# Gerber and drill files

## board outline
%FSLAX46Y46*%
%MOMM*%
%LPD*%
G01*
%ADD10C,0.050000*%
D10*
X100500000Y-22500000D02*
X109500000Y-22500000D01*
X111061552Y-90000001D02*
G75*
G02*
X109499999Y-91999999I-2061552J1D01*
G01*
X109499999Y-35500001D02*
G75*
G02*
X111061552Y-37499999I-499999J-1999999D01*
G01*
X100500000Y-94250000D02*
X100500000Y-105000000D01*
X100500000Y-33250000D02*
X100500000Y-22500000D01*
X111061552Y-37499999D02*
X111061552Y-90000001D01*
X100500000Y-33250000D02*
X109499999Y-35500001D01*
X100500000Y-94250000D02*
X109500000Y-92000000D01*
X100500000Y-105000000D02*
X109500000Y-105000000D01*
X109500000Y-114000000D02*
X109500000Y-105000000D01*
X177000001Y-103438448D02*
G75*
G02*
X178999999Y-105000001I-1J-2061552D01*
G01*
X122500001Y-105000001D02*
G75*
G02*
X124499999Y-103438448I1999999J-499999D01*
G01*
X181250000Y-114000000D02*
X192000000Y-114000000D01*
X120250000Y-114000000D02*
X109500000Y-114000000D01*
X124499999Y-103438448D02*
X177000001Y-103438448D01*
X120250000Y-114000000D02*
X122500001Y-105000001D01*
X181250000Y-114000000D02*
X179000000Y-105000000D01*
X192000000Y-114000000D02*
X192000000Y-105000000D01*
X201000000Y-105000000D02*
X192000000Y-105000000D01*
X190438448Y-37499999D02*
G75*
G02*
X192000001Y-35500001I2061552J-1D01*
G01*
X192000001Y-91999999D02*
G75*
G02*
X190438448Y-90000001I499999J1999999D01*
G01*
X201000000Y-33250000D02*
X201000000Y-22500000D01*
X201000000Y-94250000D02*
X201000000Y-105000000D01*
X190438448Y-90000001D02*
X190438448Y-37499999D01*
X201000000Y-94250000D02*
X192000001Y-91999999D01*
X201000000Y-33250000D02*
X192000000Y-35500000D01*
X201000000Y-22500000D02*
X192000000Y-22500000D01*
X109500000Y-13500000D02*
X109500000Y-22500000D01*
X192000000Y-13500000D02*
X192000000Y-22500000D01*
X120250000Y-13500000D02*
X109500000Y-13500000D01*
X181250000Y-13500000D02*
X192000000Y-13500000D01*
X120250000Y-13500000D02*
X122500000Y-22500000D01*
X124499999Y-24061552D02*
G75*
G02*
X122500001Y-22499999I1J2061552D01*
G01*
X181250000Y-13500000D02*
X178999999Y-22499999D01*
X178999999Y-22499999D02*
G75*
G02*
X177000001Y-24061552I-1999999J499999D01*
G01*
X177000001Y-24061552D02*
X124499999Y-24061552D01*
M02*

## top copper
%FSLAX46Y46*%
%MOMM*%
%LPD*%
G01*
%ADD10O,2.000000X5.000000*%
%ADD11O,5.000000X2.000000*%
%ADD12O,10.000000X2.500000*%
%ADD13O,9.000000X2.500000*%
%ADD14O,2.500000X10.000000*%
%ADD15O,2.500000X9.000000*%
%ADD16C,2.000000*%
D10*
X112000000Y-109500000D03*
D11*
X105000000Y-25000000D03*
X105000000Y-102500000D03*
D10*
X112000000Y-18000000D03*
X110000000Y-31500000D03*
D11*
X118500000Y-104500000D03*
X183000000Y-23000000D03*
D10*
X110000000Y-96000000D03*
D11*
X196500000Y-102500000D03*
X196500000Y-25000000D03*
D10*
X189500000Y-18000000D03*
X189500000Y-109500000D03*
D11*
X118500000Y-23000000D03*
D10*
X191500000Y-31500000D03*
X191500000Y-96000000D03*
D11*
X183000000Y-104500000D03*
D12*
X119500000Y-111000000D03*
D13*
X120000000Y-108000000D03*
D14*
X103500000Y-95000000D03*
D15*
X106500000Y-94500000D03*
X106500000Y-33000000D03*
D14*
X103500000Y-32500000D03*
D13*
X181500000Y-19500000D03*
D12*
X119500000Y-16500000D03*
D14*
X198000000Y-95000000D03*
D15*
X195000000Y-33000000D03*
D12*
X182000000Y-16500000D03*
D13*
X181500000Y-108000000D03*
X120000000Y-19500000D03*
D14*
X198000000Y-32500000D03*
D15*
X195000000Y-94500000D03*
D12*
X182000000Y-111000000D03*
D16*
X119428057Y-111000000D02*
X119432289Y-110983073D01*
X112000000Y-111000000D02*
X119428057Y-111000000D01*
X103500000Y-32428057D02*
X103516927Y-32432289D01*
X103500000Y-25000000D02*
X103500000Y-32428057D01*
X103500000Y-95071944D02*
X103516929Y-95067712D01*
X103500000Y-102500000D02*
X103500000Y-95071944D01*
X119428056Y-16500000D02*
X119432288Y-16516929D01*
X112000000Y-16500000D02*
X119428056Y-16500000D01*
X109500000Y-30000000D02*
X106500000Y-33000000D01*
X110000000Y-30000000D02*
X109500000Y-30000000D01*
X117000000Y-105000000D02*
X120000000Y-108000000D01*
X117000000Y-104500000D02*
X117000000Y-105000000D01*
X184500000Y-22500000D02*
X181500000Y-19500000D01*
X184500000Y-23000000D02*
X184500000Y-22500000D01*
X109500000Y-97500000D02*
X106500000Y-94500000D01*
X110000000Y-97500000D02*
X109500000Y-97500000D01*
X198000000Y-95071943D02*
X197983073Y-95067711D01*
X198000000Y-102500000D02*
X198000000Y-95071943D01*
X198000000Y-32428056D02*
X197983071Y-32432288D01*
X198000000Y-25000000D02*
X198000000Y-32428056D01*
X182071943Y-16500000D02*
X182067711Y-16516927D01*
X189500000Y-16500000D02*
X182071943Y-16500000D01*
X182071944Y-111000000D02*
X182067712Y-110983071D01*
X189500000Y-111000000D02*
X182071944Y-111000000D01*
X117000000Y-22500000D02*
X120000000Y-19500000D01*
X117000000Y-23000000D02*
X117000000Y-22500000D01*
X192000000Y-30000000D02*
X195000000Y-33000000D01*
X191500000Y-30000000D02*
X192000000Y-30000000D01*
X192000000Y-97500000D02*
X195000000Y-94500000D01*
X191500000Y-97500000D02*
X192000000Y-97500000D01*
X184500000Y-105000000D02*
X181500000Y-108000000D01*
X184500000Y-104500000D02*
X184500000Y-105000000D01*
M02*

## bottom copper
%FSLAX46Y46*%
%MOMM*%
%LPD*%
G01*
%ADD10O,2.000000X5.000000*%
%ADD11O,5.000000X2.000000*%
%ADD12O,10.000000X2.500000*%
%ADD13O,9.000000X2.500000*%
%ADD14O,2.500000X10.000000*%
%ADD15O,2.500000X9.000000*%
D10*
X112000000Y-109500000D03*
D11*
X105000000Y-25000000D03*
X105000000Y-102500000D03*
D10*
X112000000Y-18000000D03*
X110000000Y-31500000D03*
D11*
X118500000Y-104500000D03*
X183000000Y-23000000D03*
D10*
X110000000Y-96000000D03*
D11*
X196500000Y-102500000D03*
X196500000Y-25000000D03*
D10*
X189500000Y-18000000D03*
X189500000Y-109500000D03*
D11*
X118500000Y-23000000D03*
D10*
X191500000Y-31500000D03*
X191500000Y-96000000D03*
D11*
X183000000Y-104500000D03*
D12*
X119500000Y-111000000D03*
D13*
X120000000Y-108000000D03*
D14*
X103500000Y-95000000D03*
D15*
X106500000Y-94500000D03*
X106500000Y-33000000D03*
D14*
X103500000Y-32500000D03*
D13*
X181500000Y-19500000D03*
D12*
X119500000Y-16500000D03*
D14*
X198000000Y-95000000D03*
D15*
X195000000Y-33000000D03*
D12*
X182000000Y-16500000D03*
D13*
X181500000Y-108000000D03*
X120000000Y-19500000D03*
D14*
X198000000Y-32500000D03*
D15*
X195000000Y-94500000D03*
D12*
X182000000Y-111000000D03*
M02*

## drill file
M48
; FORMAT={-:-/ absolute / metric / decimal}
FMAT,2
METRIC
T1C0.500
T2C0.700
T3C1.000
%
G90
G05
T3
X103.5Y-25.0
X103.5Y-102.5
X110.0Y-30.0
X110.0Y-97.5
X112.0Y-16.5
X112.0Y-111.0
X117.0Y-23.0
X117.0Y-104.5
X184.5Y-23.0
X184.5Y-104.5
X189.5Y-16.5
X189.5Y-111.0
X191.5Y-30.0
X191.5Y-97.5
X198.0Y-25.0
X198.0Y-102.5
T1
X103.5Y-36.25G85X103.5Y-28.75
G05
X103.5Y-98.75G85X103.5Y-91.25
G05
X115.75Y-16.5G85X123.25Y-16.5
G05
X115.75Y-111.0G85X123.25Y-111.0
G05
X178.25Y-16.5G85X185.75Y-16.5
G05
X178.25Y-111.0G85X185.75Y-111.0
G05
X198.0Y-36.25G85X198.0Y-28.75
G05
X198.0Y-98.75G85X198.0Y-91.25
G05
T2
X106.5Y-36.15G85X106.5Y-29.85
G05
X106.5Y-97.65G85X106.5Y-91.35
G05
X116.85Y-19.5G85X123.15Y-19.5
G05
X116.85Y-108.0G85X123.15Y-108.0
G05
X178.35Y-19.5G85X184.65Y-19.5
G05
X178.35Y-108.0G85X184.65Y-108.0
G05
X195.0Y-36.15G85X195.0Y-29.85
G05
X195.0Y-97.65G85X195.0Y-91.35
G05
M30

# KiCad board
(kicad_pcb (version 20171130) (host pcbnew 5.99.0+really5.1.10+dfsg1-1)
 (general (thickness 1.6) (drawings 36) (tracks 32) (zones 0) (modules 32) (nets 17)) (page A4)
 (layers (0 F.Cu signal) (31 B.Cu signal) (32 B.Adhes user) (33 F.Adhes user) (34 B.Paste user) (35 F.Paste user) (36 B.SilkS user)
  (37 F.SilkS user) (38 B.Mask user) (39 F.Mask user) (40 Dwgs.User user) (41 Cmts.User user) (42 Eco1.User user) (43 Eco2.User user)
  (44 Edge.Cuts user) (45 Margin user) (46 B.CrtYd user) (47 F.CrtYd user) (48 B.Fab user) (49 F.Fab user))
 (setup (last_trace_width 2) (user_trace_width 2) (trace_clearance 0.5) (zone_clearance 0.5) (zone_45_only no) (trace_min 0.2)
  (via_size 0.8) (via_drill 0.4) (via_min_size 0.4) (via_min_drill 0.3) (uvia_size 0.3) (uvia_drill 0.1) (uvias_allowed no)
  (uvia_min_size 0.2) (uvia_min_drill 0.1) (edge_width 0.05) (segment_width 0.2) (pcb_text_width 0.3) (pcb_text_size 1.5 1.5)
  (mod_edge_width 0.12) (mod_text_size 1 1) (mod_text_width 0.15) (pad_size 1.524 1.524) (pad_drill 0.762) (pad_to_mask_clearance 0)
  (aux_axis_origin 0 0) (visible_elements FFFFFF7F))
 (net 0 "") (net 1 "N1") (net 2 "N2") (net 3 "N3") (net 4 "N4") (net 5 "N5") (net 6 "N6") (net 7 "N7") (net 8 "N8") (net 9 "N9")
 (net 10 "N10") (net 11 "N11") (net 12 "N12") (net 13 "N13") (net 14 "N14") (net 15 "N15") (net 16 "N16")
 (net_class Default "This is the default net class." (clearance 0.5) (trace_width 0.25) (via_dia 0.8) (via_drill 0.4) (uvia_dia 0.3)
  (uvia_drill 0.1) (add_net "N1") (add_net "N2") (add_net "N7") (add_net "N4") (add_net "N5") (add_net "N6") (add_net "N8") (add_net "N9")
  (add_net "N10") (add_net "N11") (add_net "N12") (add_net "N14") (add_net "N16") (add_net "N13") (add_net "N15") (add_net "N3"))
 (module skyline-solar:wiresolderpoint (layer F.Cu) (at 112 111)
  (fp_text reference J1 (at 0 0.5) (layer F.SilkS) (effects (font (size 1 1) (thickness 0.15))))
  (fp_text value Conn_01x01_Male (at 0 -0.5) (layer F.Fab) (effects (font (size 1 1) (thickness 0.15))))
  (pad 1 thru_hole oval (at 0 0) (size 2 5) (drill 1 (offset 0 -1.5)) (layers *.Cu *.Mask) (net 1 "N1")))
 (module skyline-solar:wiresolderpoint (layer F.Cu) (at 103.5 25 270)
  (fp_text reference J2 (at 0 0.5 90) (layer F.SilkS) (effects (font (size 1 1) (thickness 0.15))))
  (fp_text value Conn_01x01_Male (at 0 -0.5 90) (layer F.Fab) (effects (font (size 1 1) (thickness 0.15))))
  (pad 1 thru_hole oval (at 0 0 270) (size 2 5) (drill 1 (offset 0 -1.5)) (layers *.Cu *.Mask) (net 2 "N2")))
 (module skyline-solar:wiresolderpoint (layer F.Cu) (at 103.5 102.5 270)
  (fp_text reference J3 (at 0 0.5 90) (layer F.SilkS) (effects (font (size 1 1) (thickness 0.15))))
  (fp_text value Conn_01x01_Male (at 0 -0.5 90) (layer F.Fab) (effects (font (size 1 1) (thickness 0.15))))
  (pad 1 thru_hole oval (at 0 0 270) (size 2 5) (drill 1 (offset 0 -1.5)) (layers *.Cu *.Mask) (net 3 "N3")))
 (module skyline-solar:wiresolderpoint (layer F.Cu) (at 112 16.5 180)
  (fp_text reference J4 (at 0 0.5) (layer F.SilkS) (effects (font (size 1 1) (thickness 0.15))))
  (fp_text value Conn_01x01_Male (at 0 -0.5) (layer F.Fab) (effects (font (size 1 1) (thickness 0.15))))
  (pad 1 thru_hole oval (at 0 0 180) (size 2 5) (drill 1 (offset 0 -1.5)) (layers *.Cu *.Mask) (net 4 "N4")))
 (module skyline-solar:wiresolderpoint (layer F.Cu) (at 110 30 180)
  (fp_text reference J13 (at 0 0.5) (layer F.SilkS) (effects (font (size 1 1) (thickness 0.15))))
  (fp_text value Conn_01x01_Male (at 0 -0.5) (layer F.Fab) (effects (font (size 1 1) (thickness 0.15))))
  (pad 1 thru_hole oval (at 0 0 180) (size 2 5) (drill 1 (offset 0 -1.5)) (layers *.Cu *.Mask) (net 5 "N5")))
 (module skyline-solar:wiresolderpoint (layer F.Cu) (at 117 104.5 270)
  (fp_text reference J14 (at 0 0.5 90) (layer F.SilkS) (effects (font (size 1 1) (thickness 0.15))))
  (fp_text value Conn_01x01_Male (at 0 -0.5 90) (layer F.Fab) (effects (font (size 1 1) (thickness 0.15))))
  (pad 1 thru_hole oval (at 0 0 270) (size 2 5) (drill 1 (offset 0 -1.5)) (layers *.Cu *.Mask) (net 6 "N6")))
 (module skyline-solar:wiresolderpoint (layer F.Cu) (at 184.5 23 90)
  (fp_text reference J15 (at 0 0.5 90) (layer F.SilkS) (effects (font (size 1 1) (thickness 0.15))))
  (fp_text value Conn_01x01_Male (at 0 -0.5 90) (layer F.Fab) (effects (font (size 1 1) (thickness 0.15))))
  (pad 1 thru_hole oval (at 0 0 90) (size 2 5) (drill 1 (offset 0 -1.5)) (layers *.Cu *.Mask) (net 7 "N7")))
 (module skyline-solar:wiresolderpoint (layer F.Cu) (at 110 97.5)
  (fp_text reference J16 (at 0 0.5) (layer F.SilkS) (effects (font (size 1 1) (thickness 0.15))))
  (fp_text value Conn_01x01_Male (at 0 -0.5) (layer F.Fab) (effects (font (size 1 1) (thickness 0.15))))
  (pad 1 thru_hole oval (at 0 0) (size 2 5) (drill 1 (offset 0 -1.5)) (layers *.Cu *.Mask) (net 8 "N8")))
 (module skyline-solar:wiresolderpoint (layer F.Cu) (at 198 102.5 90)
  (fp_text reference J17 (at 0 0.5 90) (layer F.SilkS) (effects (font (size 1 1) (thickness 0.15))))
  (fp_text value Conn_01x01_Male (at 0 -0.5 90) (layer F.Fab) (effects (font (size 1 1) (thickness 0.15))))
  (pad 1 thru_hole oval (at 0 0 90) (size 2 5) (drill 1 (offset 0 -1.5)) (layers *.Cu *.Mask) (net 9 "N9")))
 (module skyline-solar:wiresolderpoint (layer F.Cu) (at 198 25 90)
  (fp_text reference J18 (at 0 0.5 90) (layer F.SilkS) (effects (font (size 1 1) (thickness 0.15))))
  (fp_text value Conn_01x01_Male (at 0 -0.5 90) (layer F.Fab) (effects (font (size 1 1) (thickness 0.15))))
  (pad 1 thru_hole oval (at 0 0 90) (size 2 5) (drill 1 (offset 0 -1.5)) (layers *.Cu *.Mask) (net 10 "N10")))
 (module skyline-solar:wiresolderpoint (layer F.Cu) (at 189.5 16.5 180)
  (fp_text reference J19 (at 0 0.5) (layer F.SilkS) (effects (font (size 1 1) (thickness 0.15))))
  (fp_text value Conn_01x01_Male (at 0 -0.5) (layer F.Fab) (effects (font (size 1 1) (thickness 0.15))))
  (pad 1 thru_hole oval (at 0 0 180) (size 2 5) (drill 1 (offset 0 -1.5)) (layers *.Cu *.Mask) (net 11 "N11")))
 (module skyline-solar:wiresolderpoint (layer F.Cu) (at 189.5 111)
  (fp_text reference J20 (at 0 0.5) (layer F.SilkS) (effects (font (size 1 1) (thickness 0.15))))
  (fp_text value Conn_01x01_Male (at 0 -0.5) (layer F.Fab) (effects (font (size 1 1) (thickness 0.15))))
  (pad 1 thru_hole oval (at 0 0) (size 2 5) (drill 1 (offset 0 -1.5)) (layers *.Cu *.Mask) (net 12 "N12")))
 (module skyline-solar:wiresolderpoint (layer F.Cu) (at 117 23 270)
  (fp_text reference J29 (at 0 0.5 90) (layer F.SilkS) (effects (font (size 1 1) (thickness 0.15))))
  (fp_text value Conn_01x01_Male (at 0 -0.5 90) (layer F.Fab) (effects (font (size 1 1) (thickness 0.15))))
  (pad 1 thru_hole oval (at 0 0 270) (size 2 5) (drill 1 (offset 0 -1.5)) (layers *.Cu *.Mask) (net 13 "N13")))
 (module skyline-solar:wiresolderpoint (layer F.Cu) (at 191.5 30 180)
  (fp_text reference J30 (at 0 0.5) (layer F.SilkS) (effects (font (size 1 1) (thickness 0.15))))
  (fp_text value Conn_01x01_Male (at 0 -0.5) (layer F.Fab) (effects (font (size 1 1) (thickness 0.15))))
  (pad 1 thru_hole oval (at 0 0 180) (size 2 5) (drill 1 (offset 0 -1.5)) (layers *.Cu *.Mask) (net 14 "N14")))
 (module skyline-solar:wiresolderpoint (layer F.Cu) (at 191.5 97.5)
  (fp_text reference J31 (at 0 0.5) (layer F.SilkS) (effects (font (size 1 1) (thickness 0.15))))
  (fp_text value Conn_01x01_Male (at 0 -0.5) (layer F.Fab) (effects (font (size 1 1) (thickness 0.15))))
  (pad 1 thru_hole oval (at 0 0) (size 2 5) (drill 1 (offset 0 -1.5)) (layers *.Cu *.Mask) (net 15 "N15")))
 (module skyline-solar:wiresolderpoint (layer F.Cu) (at 184.5 104.5 90)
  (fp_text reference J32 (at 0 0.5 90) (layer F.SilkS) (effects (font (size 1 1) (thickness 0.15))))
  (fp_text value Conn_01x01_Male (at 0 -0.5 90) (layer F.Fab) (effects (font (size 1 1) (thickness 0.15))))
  (pad 1 thru_hole oval (at 0 0 90) (size 2 5) (drill 1 (offset 0 -1.5)) (layers *.Cu *.Mask) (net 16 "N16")))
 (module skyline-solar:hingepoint (layer F.Cu) (at 119.5 111)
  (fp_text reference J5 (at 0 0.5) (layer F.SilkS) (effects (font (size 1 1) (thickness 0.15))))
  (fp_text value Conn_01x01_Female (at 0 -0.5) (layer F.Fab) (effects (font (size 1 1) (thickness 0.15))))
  (pad 1 thru_hole oval (at 0 0) (size 10 2.5) (drill oval 8 0.5) (layers *.Cu *.Mask) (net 1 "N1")))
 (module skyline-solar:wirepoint (layer F.Cu) (at 120 108)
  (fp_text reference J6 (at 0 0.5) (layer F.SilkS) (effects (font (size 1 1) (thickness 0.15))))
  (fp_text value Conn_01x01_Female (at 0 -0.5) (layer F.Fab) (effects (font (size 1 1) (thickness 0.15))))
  (pad 1 thru_hole oval (at 0 0) (size 9 2.5) (drill oval 7 0.7) (layers *.Cu *.Mask) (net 6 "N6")))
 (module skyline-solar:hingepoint (layer F.Cu) (at 103.5 95 90)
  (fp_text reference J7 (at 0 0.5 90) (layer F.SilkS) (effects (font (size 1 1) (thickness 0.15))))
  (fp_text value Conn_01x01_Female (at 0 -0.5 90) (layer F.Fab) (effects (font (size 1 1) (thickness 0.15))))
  (pad 1 thru_hole oval (at 0 0 90) (size 10 2.5) (drill oval 8 0.5) (layers *.Cu *.Mask) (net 3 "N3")))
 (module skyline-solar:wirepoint (layer F.Cu) (at 106.5 94.5 90)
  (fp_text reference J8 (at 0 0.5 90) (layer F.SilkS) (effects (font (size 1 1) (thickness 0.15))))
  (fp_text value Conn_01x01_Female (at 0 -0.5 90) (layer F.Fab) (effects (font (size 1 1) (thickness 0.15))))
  (pad 1 thru_hole oval (at 0 0 90) (size 9 2.5) (drill oval 7 0.7) (layers *.Cu *.Mask) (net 8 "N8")))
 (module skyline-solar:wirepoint (layer F.Cu) (at 106.5 33 90)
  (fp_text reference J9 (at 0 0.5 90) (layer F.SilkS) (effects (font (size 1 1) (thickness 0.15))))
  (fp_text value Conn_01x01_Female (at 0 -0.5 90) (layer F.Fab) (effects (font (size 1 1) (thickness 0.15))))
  (pad 1 thru_hole oval (at 0 0 90) (size 9 2.5) (drill oval 7 0.7) (layers *.Cu *.Mask) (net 5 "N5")))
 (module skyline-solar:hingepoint (layer F.Cu) (at 103.5 32.5 90)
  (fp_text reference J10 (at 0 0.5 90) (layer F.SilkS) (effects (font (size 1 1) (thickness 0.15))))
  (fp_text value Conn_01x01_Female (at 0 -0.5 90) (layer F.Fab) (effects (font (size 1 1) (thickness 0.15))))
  (pad 1 thru_hole oval (at 0 0 90) (size 10 2.5) (drill oval 8 0.5) (layers *.Cu *.Mask) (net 2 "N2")))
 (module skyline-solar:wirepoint (layer F.Cu) (at 181.5 19.5)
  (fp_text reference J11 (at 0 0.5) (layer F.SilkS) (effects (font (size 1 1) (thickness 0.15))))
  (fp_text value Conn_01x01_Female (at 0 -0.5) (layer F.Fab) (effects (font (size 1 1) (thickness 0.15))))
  (pad 1 thru_hole oval (at 0 0) (size 9 2.5) (drill oval 7 0.7) (layers *.Cu *.Mask) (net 7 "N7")))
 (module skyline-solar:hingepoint (layer F.Cu) (at 119.5 16.5)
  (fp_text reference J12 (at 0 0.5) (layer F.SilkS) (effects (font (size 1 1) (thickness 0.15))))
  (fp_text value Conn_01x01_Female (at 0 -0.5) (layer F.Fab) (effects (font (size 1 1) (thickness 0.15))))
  (pad 1 thru_hole oval (at 0 0) (size 10 2.5) (drill oval 8 0.5) (layers *.Cu *.Mask) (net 4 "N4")))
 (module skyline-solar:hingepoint (layer F.Cu) (at 198 95 90)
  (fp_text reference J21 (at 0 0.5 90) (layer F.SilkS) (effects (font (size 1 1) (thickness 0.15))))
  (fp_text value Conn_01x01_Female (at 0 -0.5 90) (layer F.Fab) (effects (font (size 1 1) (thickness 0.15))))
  (pad 1 thru_hole oval (at 0 0 90) (size 10 2.5) (drill oval 8 0.5) (layers *.Cu *.Mask) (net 9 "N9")))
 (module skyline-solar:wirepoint (layer F.Cu) (at 195 33 90)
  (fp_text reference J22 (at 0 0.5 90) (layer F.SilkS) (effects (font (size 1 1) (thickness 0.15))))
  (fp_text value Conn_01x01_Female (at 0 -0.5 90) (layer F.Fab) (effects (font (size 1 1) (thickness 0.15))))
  (pad 1 thru_hole oval (at 0 0 90) (size 9 2.5) (drill oval 7 0.7) (layers *.Cu *.Mask) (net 14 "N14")))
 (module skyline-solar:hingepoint (layer F.Cu) (at 182 16.5)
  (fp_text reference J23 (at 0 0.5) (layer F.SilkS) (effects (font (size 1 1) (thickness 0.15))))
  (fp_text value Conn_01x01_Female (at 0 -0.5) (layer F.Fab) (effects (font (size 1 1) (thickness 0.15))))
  (pad 1 thru_hole oval (at 0 0) (size 10 2.5) (drill oval 8 0.5) (layers *.Cu *.Mask) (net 11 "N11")))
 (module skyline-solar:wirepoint (layer F.Cu) (at 181.5 108)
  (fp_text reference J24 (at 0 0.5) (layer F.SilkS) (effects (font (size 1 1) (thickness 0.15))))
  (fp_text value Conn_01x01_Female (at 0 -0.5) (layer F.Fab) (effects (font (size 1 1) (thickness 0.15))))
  (pad 1 thru_hole oval (at 0 0) (size 9 2.5) (drill oval 7 0.7) (layers *.Cu *.Mask) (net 16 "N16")))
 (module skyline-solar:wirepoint (layer F.Cu) (at 120 19.5)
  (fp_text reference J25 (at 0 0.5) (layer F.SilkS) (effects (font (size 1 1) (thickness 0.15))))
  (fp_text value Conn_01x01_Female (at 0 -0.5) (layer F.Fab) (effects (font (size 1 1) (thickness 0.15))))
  (pad 1 thru_hole oval (at 0 0) (size 9 2.5) (drill oval 7 0.7) (layers *.Cu *.Mask) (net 13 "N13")))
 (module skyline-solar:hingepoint (layer F.Cu) (at 198 32.5 90)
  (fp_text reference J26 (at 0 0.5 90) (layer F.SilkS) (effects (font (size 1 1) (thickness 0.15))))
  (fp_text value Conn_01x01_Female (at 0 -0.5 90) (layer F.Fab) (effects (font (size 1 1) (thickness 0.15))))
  (pad 1 thru_hole oval (at 0 0 90) (size 10 2.5) (drill oval 8 0.5) (layers *.Cu *.Mask) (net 10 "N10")))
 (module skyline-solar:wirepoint (layer F.Cu) (at 195 94.5 90)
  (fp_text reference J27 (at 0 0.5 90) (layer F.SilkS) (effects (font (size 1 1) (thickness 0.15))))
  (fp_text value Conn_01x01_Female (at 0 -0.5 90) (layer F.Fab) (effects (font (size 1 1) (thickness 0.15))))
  (pad 1 thru_hole oval (at 0 0 90) (size 9 2.5) (drill oval 7 0.7) (layers *.Cu *.Mask) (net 15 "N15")))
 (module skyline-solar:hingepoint (layer F.Cu) (at 182 111)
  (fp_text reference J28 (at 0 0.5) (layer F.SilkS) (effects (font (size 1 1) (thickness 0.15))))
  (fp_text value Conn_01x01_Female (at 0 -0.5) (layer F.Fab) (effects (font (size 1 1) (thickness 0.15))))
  (pad 1 thru_hole oval (at 0 0) (size 10 2.5) (drill oval 8 0.5) (layers *.Cu *.Mask) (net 12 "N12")))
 (gr_line (start 100.5 22.5) (end 109.5 22.5) (layer Edge.Cuts) (width 0.05))
 (gr_arc (start 109 90) (end 109.499999 91.999999) (angle -75.96375653) (layer Edge.Cuts) (width 0.05))
 (gr_arc (start 109 37.5) (end 109.499999 35.500001) (angle 75.96375653) (layer Edge.Cuts) (width 0.05))
 (gr_line (start 100.5 94.25) (end 100.5 105) (layer Edge.Cuts) (width 0.05))
 (gr_line (start 100.5 33.25) (end 100.5 22.5) (layer Edge.Cuts) (width 0.05))
 (gr_line (start 111.061552 37.499999) (end 111.061552 90.000001) (layer Edge.Cuts) (width 0.05))
 (gr_line (start 100.5 33.25) (end 109.499999 35.500001) (layer Edge.Cuts) (width 0.05))
 (gr_line (start 100.5 94.25) (end 109.5 92) (layer Edge.Cuts) (width 0.05))
 (gr_line (start 100.5 105) (end 109.5 105) (layer Edge.Cuts) (width 0.05))
 (gr_line (start 109.5 114) (end 109.5 105) (layer Edge.Cuts) (width 0.05))
 (gr_arc (start 177 105.5) (end 178.999999 105.000001) (angle -75.96375653) (layer Edge.Cuts) (width 0.05))
 (gr_arc (start 124.5 105.5) (end 122.500001 105.000001) (angle 75.96375653) (layer Edge.Cuts) (width 0.05))
 (gr_line (start 181.25 114) (end 192 114) (layer Edge.Cuts) (width 0.05))
 (gr_line (start 120.25 114) (end 109.5 114) (layer Edge.Cuts) (width 0.05))
 (gr_line (start 124.499999 103.438448) (end 177.000001 103.438448) (layer Edge.Cuts) (width 0.05))
 (gr_line (start 120.25 114) (end 122.500001 105.000001) (layer Edge.Cuts) (width 0.05))
 (gr_line (start 181.25 114) (end 179 105) (layer Edge.Cuts) (width 0.05))
 (gr_line (start 192 114) (end 192 105) (layer Edge.Cuts) (width 0.05))
 (gr_line (start 201 105) (end 192 105) (layer Edge.Cuts) (width 0.05))
 (gr_arc (start 192.5 37.5) (end 192.000001 35.500001) (angle -75.96375653) (layer Edge.Cuts) (width 0.05))
 (gr_arc (start 192.5 90) (end 192.000001 91.999999) (angle 75.96375653) (layer Edge.Cuts) (width 0.05))
 (gr_line (start 201 33.25) (end 201 22.5) (layer Edge.Cuts) (width 0.05))
 (gr_line (start 201 94.25) (end 201 105) (layer Edge.Cuts) (width 0.05))
 (gr_line (start 190.438448 90.000001) (end 190.438448 37.499999) (layer Edge.Cuts) (width 0.05))
 (gr_line (start 201 94.25) (end 192.000001 91.999999) (layer Edge.Cuts) (width 0.05))
 (gr_line (start 201 33.25) (end 192 35.5) (layer Edge.Cuts) (width 0.05))
 (gr_line (start 201 22.5) (end 192 22.5) (layer Edge.Cuts) (width 0.05))
 (gr_line (start 109.5 13.5) (end 109.5 22.5) (layer Edge.Cuts) (width 0.05))
 (gr_line (start 192 13.5) (end 192 22.5) (layer Edge.Cuts) (width 0.05))
 (gr_line (start 120.25 13.5) (end 109.5 13.5) (layer Edge.Cuts) (width 0.05))
 (gr_line (start 181.25 13.5) (end 192 13.5) (layer Edge.Cuts) (width 0.05))
 (gr_line (start 120.25 13.5) (end 122.5 22.5) (layer Edge.Cuts) (width 0.05))
 (gr_arc (start 124.5 22) (end 122.500001 22.499999) (angle -75.96375653) (layer Edge.Cuts) (width 0.05))
 (gr_line (start 181.25 13.5) (end 178.999999 22.499999) (layer Edge.Cuts) (width 0.05))
 (gr_arc (start 177 22) (end 178.999999 22.499999) (angle 75.96375653) (layer Edge.Cuts) (width 0.05))
 (gr_line (start 177.000001 24.061552) (end 124.499999 24.061552) (layer Edge.Cuts) (width 0.05))
 (segment (start 119.428057 111) (end 119.432289 110.983073) (width 2) (layer F.Cu) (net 1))
 (segment (start 112 111) (end 119.428057 111) (width 2) (layer F.Cu) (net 1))
 (segment (start 103.5 32.428057) (end 103.516927 32.432289) (width 2) (layer F.Cu) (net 2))
 (segment (start 103.5 25) (end 103.5 32.428057) (width 2) (layer F.Cu) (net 2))
 (segment (start 103.5 95.071944) (end 103.516929 95.067712) (width 2) (layer F.Cu) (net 3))
 (segment (start 103.5 102.5) (end 103.5 95.071944) (width 2) (layer F.Cu) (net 3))
 (segment (start 119.428056 16.5) (end 119.432288 16.516929) (width 2) (layer F.Cu) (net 4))
 (segment (start 112 16.5) (end 119.428056 16.5) (width 2) (layer F.Cu) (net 4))
 (segment (start 109.5 30) (end 106.5 33) (width 2) (layer F.Cu) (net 5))
 (segment (start 110 30) (end 109.5 30) (width 2) (layer F.Cu) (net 5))
 (segment (start 117 105) (end 120 108) (width 2) (layer F.Cu) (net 6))
 (segment (start 117 104.5) (end 117 105) (width 2) (layer F.Cu) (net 6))
 (segment (start 184.5 22.5) (end 181.5 19.5) (width 2) (layer F.Cu) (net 7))
 (segment (start 184.5 23) (end 184.5 22.5) (width 2) (layer F.Cu) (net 7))
 (segment (start 109.5 97.5) (end 106.5 94.5) (width 2) (layer F.Cu) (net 8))
 (segment (start 110 97.5) (end 109.5 97.5) (width 2) (layer F.Cu) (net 8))
 (segment (start 198 95.071943) (end 197.983073 95.067711) (width 2) (layer F.Cu) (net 9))
 (segment (start 198 102.5) (end 198 95.071943) (width 2) (layer F.Cu) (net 9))
 (segment (start 198 32.428056) (end 197.983071 32.432288) (width 2) (layer F.Cu) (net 10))
 (segment (start 198 25) (end 198 32.428056) (width 2) (layer F.Cu) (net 10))
 (segment (start 182.071943 16.5) (end 182.067711 16.516927) (width 2) (layer F.Cu) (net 11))
 (segment (start 189.5 16.5) (end 182.071943 16.5) (width 2) (layer F.Cu) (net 11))
 (segment (start 182.071944 111) (end 182.067712 110.983071) (width 2) (layer F.Cu) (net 12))
 (segment (start 189.5 111) (end 182.071944 111) (width 2) (layer F.Cu) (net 12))
 (segment (start 117 22.5) (end 120 19.5) (width 2) (layer F.Cu) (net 13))
 (segment (start 117 23) (end 117 22.5) (width 2) (layer F.Cu) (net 13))
 (segment (start 192 30) (end 195 33) (width 2) (layer F.Cu) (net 14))
 (segment (start 191.5 30) (end 192 30) (width 2) (layer F.Cu) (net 14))
 (segment (start 192 97.5) (end 195 94.5) (width 2) (layer F.Cu) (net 15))
 (segment (start 191.5 97.5) (end 192 97.5) (width 2) (layer F.Cu) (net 15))
 (segment (start 184.5 105) (end 181.5 108) (width 2) (layer F.Cu) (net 16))
 (segment (start 184.5 104.5) (end 184.5 105) (width 2) (layer F.Cu) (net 16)))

